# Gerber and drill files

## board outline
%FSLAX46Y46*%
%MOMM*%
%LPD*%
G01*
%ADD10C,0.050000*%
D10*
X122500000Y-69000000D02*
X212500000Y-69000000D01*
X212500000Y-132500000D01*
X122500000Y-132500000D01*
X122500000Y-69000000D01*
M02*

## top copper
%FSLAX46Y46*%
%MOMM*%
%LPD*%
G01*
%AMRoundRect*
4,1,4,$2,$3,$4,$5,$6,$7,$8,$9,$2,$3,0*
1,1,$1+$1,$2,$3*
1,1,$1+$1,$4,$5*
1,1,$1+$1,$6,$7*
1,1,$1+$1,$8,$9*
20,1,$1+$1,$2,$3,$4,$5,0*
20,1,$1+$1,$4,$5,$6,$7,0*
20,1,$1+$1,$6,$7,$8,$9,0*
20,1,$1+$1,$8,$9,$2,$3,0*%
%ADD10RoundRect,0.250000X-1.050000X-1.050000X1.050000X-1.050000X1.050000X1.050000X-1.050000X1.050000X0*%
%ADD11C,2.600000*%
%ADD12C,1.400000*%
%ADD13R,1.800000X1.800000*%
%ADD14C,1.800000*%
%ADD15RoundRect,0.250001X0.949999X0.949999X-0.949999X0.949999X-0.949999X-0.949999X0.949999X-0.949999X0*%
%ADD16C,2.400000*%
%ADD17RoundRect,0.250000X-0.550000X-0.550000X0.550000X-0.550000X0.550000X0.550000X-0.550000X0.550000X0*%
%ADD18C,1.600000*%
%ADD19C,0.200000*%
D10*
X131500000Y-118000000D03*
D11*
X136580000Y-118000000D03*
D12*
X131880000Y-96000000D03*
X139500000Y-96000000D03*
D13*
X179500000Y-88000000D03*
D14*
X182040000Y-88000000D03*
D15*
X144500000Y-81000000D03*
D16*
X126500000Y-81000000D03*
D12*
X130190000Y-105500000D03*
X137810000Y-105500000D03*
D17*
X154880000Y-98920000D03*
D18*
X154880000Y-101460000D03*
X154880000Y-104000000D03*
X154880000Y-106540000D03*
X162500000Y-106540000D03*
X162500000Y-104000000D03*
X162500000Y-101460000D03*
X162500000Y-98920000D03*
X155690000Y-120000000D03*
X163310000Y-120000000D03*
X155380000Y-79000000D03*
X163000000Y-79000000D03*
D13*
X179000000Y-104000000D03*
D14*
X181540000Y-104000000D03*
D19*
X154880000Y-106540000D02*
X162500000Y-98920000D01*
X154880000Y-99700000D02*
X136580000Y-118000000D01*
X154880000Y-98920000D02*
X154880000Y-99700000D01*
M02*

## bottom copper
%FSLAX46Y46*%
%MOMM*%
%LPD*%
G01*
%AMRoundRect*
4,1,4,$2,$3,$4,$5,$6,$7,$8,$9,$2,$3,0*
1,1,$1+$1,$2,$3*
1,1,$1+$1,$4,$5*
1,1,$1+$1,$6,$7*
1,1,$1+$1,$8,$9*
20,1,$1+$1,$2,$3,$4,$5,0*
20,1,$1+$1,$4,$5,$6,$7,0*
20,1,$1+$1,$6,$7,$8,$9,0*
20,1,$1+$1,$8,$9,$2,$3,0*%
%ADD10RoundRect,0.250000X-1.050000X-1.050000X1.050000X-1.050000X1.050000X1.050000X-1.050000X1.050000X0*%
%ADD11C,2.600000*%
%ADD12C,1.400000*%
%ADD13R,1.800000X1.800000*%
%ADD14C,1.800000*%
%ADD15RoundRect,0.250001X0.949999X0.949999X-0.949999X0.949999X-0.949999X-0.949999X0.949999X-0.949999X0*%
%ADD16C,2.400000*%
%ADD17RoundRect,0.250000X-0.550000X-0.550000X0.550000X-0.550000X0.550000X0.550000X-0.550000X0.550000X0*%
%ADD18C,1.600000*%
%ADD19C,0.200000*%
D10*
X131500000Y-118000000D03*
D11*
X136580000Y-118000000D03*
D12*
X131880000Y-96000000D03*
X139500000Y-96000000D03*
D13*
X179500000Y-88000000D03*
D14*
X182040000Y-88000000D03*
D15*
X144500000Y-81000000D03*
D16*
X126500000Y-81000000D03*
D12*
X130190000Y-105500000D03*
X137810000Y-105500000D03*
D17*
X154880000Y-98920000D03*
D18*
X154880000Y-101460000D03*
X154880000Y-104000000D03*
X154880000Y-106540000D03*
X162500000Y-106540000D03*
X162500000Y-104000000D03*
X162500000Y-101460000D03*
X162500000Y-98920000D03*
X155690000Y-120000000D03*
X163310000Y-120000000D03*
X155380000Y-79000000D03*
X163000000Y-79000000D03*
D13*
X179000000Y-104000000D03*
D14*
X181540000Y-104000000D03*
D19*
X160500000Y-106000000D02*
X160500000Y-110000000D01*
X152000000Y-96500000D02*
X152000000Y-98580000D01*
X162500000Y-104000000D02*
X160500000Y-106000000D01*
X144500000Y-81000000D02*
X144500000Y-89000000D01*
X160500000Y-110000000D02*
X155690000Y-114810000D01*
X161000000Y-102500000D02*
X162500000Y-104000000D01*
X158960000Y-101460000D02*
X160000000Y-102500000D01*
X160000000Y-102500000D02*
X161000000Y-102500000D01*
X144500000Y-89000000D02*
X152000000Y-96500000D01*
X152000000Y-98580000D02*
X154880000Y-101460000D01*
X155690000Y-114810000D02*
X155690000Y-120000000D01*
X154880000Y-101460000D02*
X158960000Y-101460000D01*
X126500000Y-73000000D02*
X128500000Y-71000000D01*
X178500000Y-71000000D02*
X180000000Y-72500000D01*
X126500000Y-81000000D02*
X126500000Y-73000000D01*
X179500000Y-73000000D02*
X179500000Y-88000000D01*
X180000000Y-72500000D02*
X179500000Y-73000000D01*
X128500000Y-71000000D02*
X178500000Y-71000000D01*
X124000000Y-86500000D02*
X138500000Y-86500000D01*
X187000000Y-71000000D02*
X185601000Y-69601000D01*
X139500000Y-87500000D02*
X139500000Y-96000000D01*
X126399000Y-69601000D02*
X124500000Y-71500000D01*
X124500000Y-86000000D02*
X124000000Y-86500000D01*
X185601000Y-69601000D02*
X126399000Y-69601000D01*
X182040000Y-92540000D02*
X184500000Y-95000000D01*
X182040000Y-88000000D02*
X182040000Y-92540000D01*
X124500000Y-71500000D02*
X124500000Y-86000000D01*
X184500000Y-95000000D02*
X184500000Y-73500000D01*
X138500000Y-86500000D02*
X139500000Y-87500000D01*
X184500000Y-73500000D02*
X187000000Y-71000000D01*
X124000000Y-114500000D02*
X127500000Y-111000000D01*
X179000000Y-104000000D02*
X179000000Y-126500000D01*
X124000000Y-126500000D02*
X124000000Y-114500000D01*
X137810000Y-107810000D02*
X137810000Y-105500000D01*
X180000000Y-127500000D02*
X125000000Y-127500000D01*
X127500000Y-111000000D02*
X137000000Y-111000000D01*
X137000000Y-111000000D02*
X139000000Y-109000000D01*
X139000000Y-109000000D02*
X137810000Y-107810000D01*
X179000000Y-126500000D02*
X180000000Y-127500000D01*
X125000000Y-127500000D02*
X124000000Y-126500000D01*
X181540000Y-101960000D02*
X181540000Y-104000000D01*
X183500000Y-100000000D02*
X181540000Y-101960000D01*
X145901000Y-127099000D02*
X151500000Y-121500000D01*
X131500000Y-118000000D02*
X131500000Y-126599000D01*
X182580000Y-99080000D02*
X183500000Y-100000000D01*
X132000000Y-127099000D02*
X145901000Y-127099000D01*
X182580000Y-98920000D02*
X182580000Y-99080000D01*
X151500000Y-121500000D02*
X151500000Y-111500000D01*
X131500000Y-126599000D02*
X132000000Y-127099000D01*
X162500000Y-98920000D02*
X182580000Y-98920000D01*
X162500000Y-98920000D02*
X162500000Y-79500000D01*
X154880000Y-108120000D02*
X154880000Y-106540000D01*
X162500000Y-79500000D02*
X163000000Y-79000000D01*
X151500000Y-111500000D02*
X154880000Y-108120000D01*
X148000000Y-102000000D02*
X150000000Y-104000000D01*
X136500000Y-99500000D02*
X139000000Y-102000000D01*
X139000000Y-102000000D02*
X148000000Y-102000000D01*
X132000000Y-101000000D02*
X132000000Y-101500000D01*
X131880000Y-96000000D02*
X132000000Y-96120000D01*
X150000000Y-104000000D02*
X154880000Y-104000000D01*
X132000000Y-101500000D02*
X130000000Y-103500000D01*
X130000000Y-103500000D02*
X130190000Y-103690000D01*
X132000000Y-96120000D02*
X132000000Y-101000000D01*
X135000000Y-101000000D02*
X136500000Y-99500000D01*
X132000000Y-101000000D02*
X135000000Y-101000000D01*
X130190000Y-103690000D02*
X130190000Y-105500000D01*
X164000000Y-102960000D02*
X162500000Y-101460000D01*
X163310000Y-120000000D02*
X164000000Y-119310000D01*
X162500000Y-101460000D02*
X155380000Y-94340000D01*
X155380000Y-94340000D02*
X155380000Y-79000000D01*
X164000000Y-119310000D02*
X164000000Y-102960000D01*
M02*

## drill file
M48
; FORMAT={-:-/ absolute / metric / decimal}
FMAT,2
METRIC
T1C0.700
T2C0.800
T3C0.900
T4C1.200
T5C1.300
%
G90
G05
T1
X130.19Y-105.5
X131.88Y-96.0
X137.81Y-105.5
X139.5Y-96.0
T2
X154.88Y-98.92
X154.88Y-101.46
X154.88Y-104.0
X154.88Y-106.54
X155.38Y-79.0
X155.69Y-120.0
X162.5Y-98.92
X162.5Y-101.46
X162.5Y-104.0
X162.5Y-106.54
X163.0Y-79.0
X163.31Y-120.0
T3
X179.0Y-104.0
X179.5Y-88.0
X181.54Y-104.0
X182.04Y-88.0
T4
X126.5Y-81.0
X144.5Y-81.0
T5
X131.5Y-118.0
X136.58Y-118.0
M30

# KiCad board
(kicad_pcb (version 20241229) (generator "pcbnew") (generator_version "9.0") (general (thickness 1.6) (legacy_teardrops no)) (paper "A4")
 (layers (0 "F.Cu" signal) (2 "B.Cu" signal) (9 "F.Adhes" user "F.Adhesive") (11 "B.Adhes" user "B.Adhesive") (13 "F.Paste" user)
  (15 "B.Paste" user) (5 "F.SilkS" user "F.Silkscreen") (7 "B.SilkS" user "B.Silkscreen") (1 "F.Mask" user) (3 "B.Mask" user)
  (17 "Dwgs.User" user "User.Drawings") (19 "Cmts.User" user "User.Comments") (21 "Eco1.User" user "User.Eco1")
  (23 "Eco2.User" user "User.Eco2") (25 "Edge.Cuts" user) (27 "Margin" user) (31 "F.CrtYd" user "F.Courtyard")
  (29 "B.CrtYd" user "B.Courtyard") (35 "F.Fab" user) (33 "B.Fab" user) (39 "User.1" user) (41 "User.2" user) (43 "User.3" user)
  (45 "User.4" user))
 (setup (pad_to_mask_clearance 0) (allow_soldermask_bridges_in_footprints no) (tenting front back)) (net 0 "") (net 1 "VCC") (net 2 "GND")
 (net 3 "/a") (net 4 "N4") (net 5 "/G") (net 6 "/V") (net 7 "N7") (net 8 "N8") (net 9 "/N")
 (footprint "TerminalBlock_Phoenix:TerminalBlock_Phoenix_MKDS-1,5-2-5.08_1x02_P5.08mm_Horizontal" (layer "F.Cu") (at 131.5 118)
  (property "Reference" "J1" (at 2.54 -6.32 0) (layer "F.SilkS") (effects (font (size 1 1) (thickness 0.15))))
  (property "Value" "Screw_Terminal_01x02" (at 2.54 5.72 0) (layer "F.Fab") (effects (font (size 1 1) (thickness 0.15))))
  (pad "1" thru_hole roundrect (at 0 0) (size 2.6 2.6) (drill 1.3) (layers "*.Cu" "*.Mask") (remove_unused_layers no)
   (roundrect_rratio 0.096154) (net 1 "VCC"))
  (pad "2" thru_hole circle (at 5.08 0) (size 2.6 2.6) (drill 1.3) (layers "*.Cu" "*.Mask") (remove_unused_layers no) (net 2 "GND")))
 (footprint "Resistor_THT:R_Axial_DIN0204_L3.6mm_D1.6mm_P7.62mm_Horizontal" (layer "F.Cu") (at 131.88 96)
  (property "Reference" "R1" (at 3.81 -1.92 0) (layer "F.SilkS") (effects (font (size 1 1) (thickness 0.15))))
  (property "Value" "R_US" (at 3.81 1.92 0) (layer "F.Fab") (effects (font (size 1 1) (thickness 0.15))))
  (pad "1" thru_hole circle (at 0 0) (size 1.4 1.4) (drill 0.7) (layers "*.Cu" "*.Mask") (remove_unused_layers no) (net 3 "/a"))
  (pad "2" thru_hole circle (at 7.62 0) (size 1.4 1.4) (drill 0.7) (layers "*.Cu" "*.Mask") (remove_unused_layers no) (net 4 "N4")))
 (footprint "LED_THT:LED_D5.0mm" (layer "F.Cu") (at 179.5 88)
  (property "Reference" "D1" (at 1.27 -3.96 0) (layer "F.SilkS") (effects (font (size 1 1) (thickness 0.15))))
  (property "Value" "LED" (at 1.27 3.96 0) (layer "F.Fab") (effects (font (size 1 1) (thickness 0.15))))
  (pad "1" thru_hole rect (at 0 0) (size 1.8 1.8) (drill 0.9) (layers "*.Cu" "*.Mask") (remove_unused_layers no) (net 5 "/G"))
  (pad "2" thru_hole circle (at 2.54 0) (size 1.8 1.8) (drill 0.9) (layers "*.Cu" "*.Mask") (remove_unused_layers no) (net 4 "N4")))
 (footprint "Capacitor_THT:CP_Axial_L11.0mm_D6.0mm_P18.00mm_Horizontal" (layer "F.Cu") (at 144.5 81 180)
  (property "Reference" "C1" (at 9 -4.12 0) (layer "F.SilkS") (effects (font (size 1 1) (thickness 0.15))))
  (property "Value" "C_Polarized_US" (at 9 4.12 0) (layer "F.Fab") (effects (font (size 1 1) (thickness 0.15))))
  (pad "1" thru_hole roundrect (at 0 0 180) (size 2.4 2.4) (drill 1.2) (layers "*.Cu" "*.Mask") (remove_unused_layers no)
   (roundrect_rratio 0.104167) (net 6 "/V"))
  (pad "2" thru_hole circle (at 18 0 180) (size 2.4 2.4) (drill 1.2) (layers "*.Cu" "*.Mask") (remove_unused_layers no) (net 5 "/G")))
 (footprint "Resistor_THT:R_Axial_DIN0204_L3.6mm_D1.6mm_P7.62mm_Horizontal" (layer "F.Cu") (at 130.19 105.5)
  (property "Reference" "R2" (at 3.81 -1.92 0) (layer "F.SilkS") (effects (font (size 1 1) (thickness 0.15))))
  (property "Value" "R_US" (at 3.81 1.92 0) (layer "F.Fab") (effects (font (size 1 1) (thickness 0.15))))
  (pad "1" thru_hole circle (at 0 0) (size 1.4 1.4) (drill 0.7) (layers "*.Cu" "*.Mask") (remove_unused_layers no) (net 3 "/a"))
  (pad "2" thru_hole circle (at 7.62 0) (size 1.4 1.4) (drill 0.7) (layers "*.Cu" "*.Mask") (remove_unused_layers no) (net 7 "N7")))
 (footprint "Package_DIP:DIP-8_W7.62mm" (layer "F.Cu") (at 154.88 98.92)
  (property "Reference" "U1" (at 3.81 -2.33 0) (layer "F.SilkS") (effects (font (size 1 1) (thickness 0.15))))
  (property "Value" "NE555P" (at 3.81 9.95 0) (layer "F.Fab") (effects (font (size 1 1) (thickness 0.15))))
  (pad "1" thru_hole roundrect (at 0 0) (size 1.6 1.6) (drill 0.8) (layers "*.Cu" "*.Mask") (remove_unused_layers no)
   (roundrect_rratio 0.15625) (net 2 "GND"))
  (pad "2" thru_hole circle (at 0 2.54) (size 1.6 1.6) (drill 0.8) (layers "*.Cu" "*.Mask") (remove_unused_layers no) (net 6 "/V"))
  (pad "3" thru_hole circle (at 0 5.08) (size 1.6 1.6) (drill 0.8) (layers "*.Cu" "*.Mask") (remove_unused_layers no) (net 3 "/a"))
  (pad "4" thru_hole circle (at 0 7.62) (size 1.6 1.6) (drill 0.8) (layers "*.Cu" "*.Mask") (remove_unused_layers no) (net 1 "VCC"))
  (pad "5" thru_hole circle (at 7.62 7.62) (size 1.6 1.6) (drill 0.8) (layers "*.Cu" "*.Mask") (remove_unused_layers no) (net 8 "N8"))
  (pad "6" thru_hole circle (at 7.62 5.08) (size 1.6 1.6) (drill 0.8) (layers "*.Cu" "*.Mask") (remove_unused_layers no) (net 6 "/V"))
  (pad "7" thru_hole circle (at 7.62 2.54) (size 1.6 1.6) (drill 0.8) (layers "*.Cu" "*.Mask") (remove_unused_layers no) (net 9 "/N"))
  (pad "8" thru_hole circle (at 7.62 0) (size 1.6 1.6) (drill 0.8) (layers "*.Cu" "*.Mask") (remove_unused_layers no) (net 1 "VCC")))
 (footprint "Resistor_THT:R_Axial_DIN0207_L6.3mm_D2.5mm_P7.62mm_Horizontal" (layer "F.Cu") (at 155.69 120)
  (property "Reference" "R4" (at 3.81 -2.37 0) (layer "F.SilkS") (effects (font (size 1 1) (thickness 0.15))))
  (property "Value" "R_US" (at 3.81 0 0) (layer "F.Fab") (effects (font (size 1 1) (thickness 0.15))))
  (pad "1" thru_hole circle (at 0 0) (size 1.6 1.6) (drill 0.8) (layers "*.Cu" "*.Mask") (remove_unused_layers no) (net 6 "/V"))
  (pad "2" thru_hole circle (at 7.62 0) (size 1.6 1.6) (drill 0.8) (layers "*.Cu" "*.Mask") (remove_unused_layers no) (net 9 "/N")))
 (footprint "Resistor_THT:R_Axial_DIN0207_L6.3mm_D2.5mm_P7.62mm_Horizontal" (layer "F.Cu") (at 155.38 79)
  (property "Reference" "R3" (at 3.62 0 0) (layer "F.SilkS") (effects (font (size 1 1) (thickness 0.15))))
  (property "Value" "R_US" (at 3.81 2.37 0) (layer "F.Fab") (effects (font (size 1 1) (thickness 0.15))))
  (pad "1" thru_hole circle (at 0 0) (size 1.6 1.6) (drill 0.8) (layers "*.Cu" "*.Mask") (remove_unused_layers no) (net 9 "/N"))
  (pad "2" thru_hole circle (at 7.62 0) (size 1.6 1.6) (drill 0.8) (layers "*.Cu" "*.Mask") (remove_unused_layers no) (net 1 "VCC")))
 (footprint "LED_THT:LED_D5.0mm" (layer "F.Cu") (at 179 104)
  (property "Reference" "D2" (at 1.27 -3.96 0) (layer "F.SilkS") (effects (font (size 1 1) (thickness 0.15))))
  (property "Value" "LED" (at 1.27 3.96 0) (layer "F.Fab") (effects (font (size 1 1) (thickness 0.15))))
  (pad "1" thru_hole rect (at 0 0) (size 1.8 1.8) (drill 0.9) (layers "*.Cu" "*.Mask") (remove_unused_layers no) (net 7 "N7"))
  (pad "2" thru_hole circle (at 2.54 0) (size 1.8 1.8) (drill 0.9) (layers "*.Cu" "*.Mask") (remove_unused_layers no) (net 1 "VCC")))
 (gr_rect (start 122.5 69) (end 212.5 132.5) (stroke (width 0.05) (type default)) (fill no) (layer "Edge.Cuts"))
 (segment (start 160.5 106) (end 160.5 110) (width 0.2) (layer "B.Cu") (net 6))
 (segment (start 152 96.5) (end 152 98.58) (width 0.2) (layer "B.Cu") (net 6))
 (segment (start 162.5 104) (end 160.5 106) (width 0.2) (layer "B.Cu") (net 6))
 (segment (start 144.5 81) (end 144.5 89) (width 0.2) (layer "B.Cu") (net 6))
 (segment (start 160.5 110) (end 155.69 114.81) (width 0.2) (layer "B.Cu") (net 6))
 (segment (start 161 102.5) (end 162.5 104) (width 0.2) (layer "B.Cu") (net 6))
 (segment (start 158.96 101.46) (end 160 102.5) (width 0.2) (layer "B.Cu") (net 6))
 (segment (start 160 102.5) (end 161 102.5) (width 0.2) (layer "B.Cu") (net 6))
 (segment (start 144.5 89) (end 152 96.5) (width 0.2) (layer "B.Cu") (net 6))
 (segment (start 152 98.58) (end 154.88 101.46) (width 0.2) (layer "B.Cu") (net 6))
 (segment (start 155.69 114.81) (end 155.69 120) (width 0.2) (layer "B.Cu") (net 6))
 (segment (start 154.88 101.46) (end 158.96 101.46) (width 0.2) (layer "B.Cu") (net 6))
 (segment (start 126.5 73) (end 128.5 71) (width 0.2) (layer "B.Cu") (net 5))
 (segment (start 178.5 71) (end 180 72.5) (width 0.2) (layer "B.Cu") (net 5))
 (segment (start 126.5 81) (end 126.5 73) (width 0.2) (layer "B.Cu") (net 5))
 (segment (start 179.5 73) (end 179.5 88) (width 0.2) (layer "B.Cu") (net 5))
 (segment (start 180 72.5) (end 179.5 73) (width 0.2) (layer "B.Cu") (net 5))
 (segment (start 128.5 71) (end 178.5 71) (width 0.2) (layer "B.Cu") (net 5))
 (segment (start 124 86.5) (end 138.5 86.5) (width 0.2) (layer "B.Cu") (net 4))
 (segment (start 187 71) (end 185.601 69.601) (width 0.2) (layer "B.Cu") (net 4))
 (segment (start 139.5 87.5) (end 139.5 96) (width 0.2) (layer "B.Cu") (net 4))
 (segment (start 126.399 69.601) (end 124.5 71.5) (width 0.2) (layer "B.Cu") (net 4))
 (segment (start 124.5 86) (end 124 86.5) (width 0.2) (layer "B.Cu") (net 4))
 (segment (start 185.601 69.601) (end 126.399 69.601) (width 0.2) (layer "B.Cu") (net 4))
 (segment (start 182.04 92.54) (end 184.5 95) (width 0.2) (layer "B.Cu") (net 4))
 (segment (start 182.04 88) (end 182.04 92.54) (width 0.2) (layer "B.Cu") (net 4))
 (segment (start 124.5 71.5) (end 124.5 86) (width 0.2) (layer "B.Cu") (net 4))
 (segment (start 184.5 95) (end 184.5 73.5) (width 0.2) (layer "B.Cu") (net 4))
 (segment (start 138.5 86.5) (end 139.5 87.5) (width 0.2) (layer "B.Cu") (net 4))
 (segment (start 184.5 73.5) (end 187 71) (width 0.2) (layer "B.Cu") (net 4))
 (segment (start 124 114.5) (end 127.5 111) (width 0.2) (layer "B.Cu") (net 7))
 (segment (start 179 104) (end 179 126.5) (width 0.2) (layer "B.Cu") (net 7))
 (segment (start 124 126.5) (end 124 114.5) (width 0.2) (layer "B.Cu") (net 7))
 (segment (start 137.81 107.81) (end 137.81 105.5) (width 0.2) (layer "B.Cu") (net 7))
 (segment (start 180 127.5) (end 125 127.5) (width 0.2) (layer "B.Cu") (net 7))
 (segment (start 127.5 111) (end 137 111) (width 0.2) (layer "B.Cu") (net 7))
 (segment (start 137 111) (end 139 109) (width 0.2) (layer "B.Cu") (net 7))
 (segment (start 139 109) (end 137.81 107.81) (width 0.2) (layer "B.Cu") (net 7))
 (segment (start 179 126.5) (end 180 127.5) (width 0.2) (layer "B.Cu") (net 7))
 (segment (start 125 127.5) (end 124 126.5) (width 0.2) (layer "B.Cu") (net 7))
 (segment (start 154.88 106.54) (end 162.5 98.92) (width 0.2) (layer "F.Cu") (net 1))
 (segment (start 181.54 101.96) (end 181.54 104) (width 0.2) (layer "B.Cu") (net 1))
 (segment (start 183.5 100) (end 181.54 101.96) (width 0.2) (layer "B.Cu") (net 1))
 (segment (start 145.901 127.099) (end 151.5 121.5) (width 0.2) (layer "B.Cu") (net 1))
 (segment (start 131.5 118) (end 131.5 126.599) (width 0.2) (layer "B.Cu") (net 1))
 (segment (start 182.58 99.08) (end 183.5 100) (width 0.2) (layer "B.Cu") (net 1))
 (segment (start 132 127.099) (end 145.901 127.099) (width 0.2) (layer "B.Cu") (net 1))
 (segment (start 182.58 98.92) (end 182.58 99.08) (width 0.2) (layer "B.Cu") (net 1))
 (segment (start 151.5 121.5) (end 151.5 111.5) (width 0.2) (layer "B.Cu") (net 1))
 (segment (start 131.5 126.599) (end 132 127.099) (width 0.2) (layer "B.Cu") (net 1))
 (segment (start 162.5 98.92) (end 182.58 98.92) (width 0.2) (layer "B.Cu") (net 1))
 (segment (start 162.5 98.92) (end 162.5 79.5) (width 0.2) (layer "B.Cu") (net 1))
 (segment (start 154.88 108.12) (end 154.88 106.54) (width 0.2) (layer "B.Cu") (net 1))
 (segment (start 162.5 79.5) (end 163 79) (width 0.2) (layer "B.Cu") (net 1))
 (segment (start 151.5 111.5) (end 154.88 108.12) (width 0.2) (layer "B.Cu") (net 1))
 (segment (start 154.88 99.7) (end 136.58 118) (width 0.2) (layer "F.Cu") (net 2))
 (segment (start 154.88 98.92) (end 154.88 99.7) (width 0.2) (layer "F.Cu") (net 2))
 (segment (start 148 102) (end 150 104) (width 0.2) (layer "B.Cu") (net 3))
 (segment (start 136.5 99.5) (end 139 102) (width 0.2) (layer "B.Cu") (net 3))
 (segment (start 139 102) (end 148 102) (width 0.2) (layer "B.Cu") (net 3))
 (segment (start 132 101) (end 132 101.5) (width 0.2) (layer "B.Cu") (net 3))
 (segment (start 131.88 96) (end 132 96.12) (width 0.2) (layer "B.Cu") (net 3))
 (segment (start 150 104) (end 154.88 104) (width 0.2) (layer "B.Cu") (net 3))
 (segment (start 132 101.5) (end 130 103.5) (width 0.2) (layer "B.Cu") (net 3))
 (segment (start 130 103.5) (end 130.19 103.69) (width 0.2) (layer "B.Cu") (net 3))
 (segment (start 132 96.12) (end 132 101) (width 0.2) (layer "B.Cu") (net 3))
 (segment (start 135 101) (end 136.5 99.5) (width 0.2) (layer "B.Cu") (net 3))
 (segment (start 132 101) (end 135 101) (width 0.2) (layer "B.Cu") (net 3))
 (segment (start 130.19 103.69) (end 130.19 105.5) (width 0.2) (layer "B.Cu") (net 3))
 (segment (start 164 102.96) (end 162.5 101.46) (width 0.2) (layer "B.Cu") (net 9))
 (segment (start 163.31 120) (end 164 119.31) (width 0.2) (layer "B.Cu") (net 9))
 (segment (start 162.5 101.46) (end 155.38 94.34) (width 0.2) (layer "B.Cu") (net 9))
 (segment (start 155.38 94.34) (end 155.38 79) (width 0.2) (layer "B.Cu") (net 9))
 (segment (start 164 119.31) (end 164 102.96) (width 0.2) (layer "B.Cu") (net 9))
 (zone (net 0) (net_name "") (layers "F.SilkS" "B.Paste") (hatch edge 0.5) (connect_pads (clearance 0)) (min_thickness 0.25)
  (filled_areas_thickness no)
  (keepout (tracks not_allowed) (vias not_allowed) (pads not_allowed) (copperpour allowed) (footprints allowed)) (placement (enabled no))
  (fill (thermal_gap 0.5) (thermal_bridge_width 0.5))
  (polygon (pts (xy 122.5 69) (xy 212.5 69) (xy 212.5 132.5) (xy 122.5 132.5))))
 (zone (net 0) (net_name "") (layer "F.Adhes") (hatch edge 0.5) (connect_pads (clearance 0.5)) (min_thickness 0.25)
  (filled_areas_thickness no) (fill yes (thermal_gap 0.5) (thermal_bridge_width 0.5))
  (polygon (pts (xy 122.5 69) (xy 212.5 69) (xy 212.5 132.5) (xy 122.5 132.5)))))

